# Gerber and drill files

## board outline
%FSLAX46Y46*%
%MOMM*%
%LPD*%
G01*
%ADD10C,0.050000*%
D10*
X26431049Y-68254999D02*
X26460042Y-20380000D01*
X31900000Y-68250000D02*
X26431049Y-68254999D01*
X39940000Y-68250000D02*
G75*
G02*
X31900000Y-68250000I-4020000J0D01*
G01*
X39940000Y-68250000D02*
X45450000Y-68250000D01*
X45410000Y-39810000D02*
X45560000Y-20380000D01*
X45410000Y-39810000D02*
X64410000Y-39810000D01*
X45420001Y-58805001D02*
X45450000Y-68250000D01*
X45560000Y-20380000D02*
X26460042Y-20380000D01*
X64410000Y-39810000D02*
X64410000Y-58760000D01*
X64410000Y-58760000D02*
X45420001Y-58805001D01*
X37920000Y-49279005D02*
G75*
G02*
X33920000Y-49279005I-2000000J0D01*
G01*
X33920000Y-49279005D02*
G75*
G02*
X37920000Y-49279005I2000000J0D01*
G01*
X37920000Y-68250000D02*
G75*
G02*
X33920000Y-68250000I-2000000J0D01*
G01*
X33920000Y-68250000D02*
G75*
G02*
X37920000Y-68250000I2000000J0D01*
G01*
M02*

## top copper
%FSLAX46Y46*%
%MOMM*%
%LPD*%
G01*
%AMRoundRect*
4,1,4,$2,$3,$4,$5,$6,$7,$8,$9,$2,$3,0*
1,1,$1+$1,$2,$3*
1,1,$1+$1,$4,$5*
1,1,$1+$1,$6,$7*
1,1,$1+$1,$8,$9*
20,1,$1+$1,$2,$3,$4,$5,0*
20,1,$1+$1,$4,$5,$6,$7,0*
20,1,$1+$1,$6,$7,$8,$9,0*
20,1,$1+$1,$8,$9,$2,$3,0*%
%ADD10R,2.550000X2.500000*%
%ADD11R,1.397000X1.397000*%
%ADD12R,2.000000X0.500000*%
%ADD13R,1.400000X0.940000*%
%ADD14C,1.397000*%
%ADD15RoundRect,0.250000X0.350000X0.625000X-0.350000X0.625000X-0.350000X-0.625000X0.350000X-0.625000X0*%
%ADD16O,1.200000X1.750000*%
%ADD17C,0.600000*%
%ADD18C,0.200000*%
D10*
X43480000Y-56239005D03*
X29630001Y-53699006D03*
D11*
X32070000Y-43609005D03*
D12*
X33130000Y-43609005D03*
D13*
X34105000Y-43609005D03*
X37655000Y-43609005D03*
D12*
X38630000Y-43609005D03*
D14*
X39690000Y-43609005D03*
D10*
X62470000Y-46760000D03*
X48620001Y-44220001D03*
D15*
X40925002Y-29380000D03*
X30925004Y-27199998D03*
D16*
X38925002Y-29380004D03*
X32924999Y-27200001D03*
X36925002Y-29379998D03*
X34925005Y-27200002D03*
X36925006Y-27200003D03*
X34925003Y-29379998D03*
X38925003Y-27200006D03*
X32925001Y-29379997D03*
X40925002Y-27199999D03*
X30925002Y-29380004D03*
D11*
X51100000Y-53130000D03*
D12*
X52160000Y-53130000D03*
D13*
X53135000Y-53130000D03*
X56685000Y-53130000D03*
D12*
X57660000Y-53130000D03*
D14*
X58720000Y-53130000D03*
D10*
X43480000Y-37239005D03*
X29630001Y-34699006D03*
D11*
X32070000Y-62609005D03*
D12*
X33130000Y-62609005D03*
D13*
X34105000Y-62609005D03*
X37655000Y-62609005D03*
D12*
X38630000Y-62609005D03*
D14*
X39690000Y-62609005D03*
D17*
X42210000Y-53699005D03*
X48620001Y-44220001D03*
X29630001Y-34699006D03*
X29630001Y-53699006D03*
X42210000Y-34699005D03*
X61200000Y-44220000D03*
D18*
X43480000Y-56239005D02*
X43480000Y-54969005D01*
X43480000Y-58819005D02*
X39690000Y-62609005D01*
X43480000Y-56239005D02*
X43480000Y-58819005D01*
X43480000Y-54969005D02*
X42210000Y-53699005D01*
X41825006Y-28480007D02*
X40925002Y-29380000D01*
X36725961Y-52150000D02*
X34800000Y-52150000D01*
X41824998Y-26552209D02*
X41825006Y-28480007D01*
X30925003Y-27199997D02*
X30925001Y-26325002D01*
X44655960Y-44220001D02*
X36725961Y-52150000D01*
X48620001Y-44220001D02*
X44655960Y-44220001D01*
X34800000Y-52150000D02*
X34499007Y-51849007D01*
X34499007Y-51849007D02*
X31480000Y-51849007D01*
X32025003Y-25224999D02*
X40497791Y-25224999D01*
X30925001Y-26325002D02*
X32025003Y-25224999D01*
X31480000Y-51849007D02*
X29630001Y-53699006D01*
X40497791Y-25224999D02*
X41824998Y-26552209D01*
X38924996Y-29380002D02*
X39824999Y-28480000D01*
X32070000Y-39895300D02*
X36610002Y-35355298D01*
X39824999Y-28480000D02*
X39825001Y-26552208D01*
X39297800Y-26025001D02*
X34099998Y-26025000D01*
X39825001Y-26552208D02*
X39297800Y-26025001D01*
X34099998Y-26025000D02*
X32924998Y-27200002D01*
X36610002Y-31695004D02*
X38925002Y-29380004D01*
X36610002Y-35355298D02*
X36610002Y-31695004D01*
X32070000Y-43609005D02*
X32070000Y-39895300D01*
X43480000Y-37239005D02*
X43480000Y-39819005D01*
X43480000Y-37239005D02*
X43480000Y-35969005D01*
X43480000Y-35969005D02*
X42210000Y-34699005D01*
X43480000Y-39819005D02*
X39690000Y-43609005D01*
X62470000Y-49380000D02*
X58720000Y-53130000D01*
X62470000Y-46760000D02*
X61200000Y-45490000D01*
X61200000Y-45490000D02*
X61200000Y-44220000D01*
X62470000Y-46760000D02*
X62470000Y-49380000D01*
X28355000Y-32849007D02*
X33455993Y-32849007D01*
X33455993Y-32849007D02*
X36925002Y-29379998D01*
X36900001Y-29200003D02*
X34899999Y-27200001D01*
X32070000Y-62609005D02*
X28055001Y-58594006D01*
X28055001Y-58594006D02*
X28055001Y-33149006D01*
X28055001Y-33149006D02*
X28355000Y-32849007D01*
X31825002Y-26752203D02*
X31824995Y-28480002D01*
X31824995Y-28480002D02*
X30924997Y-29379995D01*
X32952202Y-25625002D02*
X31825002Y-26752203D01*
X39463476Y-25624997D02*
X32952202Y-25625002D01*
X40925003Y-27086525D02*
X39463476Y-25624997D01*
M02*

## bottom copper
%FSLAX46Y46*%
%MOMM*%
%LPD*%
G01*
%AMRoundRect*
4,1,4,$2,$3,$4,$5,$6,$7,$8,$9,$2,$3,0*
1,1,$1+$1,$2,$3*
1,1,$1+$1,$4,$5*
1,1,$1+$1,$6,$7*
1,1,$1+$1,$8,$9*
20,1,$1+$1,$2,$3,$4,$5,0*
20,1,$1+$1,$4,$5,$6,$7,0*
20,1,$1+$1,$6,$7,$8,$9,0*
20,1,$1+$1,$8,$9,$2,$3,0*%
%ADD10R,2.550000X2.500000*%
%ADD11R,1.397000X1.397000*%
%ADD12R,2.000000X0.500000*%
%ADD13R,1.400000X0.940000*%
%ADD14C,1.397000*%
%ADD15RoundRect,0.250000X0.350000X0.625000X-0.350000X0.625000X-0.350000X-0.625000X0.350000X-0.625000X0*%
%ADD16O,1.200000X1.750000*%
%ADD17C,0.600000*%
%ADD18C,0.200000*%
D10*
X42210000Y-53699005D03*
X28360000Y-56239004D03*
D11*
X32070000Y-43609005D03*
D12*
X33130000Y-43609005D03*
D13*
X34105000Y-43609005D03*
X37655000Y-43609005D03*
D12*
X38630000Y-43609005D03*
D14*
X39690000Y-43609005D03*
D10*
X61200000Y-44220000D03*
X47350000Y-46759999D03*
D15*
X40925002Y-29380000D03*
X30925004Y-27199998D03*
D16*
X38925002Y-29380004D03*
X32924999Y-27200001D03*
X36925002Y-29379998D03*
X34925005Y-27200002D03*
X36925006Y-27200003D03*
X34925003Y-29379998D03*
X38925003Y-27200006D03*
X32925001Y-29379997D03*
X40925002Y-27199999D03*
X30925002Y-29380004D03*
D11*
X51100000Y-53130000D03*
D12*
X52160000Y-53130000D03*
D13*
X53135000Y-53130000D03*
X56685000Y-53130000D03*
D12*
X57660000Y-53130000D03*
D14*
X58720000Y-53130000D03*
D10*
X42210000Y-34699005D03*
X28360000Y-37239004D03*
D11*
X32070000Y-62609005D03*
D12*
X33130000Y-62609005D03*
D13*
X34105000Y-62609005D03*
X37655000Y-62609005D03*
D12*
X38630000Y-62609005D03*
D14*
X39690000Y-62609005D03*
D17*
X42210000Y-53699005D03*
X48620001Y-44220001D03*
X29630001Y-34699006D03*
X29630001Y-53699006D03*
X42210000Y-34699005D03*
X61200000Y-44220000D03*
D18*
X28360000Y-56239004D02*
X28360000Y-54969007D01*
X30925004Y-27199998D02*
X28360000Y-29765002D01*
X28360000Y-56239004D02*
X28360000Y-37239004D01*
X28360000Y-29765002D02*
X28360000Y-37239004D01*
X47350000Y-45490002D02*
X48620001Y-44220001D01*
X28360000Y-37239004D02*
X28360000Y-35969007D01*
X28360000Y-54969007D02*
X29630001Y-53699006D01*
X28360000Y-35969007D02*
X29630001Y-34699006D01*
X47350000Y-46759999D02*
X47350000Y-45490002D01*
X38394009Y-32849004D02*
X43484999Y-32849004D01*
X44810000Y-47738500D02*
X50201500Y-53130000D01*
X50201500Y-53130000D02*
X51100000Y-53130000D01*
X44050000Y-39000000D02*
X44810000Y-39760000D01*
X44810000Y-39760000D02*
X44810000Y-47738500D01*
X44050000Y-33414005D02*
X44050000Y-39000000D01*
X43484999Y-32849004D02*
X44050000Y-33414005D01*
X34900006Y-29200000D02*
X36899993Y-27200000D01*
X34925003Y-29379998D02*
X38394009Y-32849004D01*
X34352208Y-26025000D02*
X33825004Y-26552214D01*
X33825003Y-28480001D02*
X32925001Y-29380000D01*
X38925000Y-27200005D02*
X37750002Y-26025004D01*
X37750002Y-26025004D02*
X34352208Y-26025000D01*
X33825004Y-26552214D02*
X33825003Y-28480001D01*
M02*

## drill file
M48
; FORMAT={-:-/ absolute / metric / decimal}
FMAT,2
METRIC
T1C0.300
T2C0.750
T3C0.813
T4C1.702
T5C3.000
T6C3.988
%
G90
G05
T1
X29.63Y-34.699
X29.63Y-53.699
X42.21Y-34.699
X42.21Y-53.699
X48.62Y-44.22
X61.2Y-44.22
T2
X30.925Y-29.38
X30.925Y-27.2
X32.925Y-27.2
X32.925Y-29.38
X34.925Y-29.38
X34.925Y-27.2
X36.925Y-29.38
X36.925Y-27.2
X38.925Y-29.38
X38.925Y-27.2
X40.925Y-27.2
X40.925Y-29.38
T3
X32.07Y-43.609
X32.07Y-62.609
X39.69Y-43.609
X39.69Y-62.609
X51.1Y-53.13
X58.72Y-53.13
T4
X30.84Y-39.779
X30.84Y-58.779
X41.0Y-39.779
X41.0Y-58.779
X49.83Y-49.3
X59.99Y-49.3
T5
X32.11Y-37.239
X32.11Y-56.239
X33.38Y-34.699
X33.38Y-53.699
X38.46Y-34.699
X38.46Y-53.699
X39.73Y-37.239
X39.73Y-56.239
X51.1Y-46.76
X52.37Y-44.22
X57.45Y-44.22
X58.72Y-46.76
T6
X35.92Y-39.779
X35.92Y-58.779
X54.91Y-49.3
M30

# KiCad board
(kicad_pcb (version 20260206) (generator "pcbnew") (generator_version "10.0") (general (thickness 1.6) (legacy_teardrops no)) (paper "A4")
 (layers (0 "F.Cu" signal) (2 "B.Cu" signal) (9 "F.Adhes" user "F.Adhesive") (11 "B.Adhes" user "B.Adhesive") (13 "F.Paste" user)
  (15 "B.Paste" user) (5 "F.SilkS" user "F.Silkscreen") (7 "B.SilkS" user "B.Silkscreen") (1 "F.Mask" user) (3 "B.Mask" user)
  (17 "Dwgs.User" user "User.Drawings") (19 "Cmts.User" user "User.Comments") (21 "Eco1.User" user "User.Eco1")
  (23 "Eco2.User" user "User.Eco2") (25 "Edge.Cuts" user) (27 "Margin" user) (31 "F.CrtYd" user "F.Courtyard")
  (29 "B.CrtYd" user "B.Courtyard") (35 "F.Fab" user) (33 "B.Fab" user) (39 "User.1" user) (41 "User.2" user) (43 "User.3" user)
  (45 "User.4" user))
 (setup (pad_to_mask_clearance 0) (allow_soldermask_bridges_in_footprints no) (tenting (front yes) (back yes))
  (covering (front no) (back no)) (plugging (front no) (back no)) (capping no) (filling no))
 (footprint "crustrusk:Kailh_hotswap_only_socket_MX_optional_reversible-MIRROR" (layer "F.Cu") (at 35.92 58.779005)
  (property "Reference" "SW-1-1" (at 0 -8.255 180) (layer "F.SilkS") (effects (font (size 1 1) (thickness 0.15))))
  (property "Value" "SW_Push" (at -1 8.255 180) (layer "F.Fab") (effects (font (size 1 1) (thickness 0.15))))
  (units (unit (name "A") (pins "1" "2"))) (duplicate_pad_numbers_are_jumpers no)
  (pad "" np_thru_hole circle (at -5.08 0) (size 1.7018 1.7018) (drill 1.7018) (layers "*.Cu" "*.Mask"))
  (pad "" np_thru_hole circle (at -3.81 -2.54 180) (size 3 3) (drill 3) (layers "*.Cu" "*.Mask"))
  (pad "" np_thru_hole circle (at -2.54 -5.079998) (size 3 3) (drill 3) (layers "*.Cu" "*.Mask"))
  (pad "" np_thru_hole circle (at 0 0) (size 3.9878 3.9878) (drill 3.9878) (layers "*.Cu" "*.Mask"))
  (pad "" np_thru_hole circle (at 2.540002 -5.080001 180) (size 3 3) (drill 3) (layers "*.Cu" "*.Mask"))
  (pad "" np_thru_hole circle (at 3.81 -2.54) (size 3 3) (drill 3) (layers "*.Cu" "*.Mask"))
  (pad "" np_thru_hole circle (at 5.08 0) (size 1.7018 1.7018) (drill 1.7018) (layers "*.Cu" "*.Mask"))
  (pad "1" smd rect (at 6.29 -5.08 180) (size 2.55 2.5) (layers "B.Cu" "B.Mask" "B.Paste") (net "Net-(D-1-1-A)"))
  (pad "1" smd rect (at 7.56 -2.54) (size 2.55 2.5) (layers "F.Cu" "F.Mask" "F.Paste") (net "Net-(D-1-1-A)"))
  (pad "2" smd rect (at -7.56 -2.540001 180) (size 2.55 2.5) (layers "B.Cu" "B.Mask" "B.Paste") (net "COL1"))
  (pad "2" smd rect (at -6.289999 -5.079999) (size 2.55 2.5) (layers "F.Cu" "F.Mask" "F.Paste") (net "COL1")))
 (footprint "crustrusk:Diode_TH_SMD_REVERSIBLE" (layer "F.Cu") (at 35.88 43.609005)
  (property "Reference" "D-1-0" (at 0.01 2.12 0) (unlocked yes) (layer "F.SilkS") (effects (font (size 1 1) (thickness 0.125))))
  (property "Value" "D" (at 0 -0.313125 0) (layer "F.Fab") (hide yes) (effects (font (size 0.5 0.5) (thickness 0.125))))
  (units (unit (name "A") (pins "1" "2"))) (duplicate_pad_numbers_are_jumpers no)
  (pad "1" thru_hole rect (at -3.81 0) (size 1.397 1.397) (drill 0.8128) (layers "*.Cu" "*.Mask") (remove_unused_layers no) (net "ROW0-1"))
  (pad "1" smd rect (at -2.75 0 180) (size 2 0.5) (layers "F.Cu") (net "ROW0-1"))
  (pad "1" smd rect (at -2.75 0) (size 2 0.5) (layers "B.Cu") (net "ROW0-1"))
  (pad "1" smd rect (at -1.775 0 180) (size 1.4 0.94) (layers "F.Cu" "F.Mask" "F.Paste") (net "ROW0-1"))
  (pad "1" smd rect (at -1.775 0) (size 1.4 0.94) (layers "B.Cu" "B.Mask" "B.Paste") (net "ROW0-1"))
  (pad "2" smd rect (at 1.775 0 180) (size 1.4 0.94) (layers "F.Cu" "F.Mask" "F.Paste") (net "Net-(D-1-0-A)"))
  (pad "2" smd rect (at 1.775 0) (size 1.4 0.94) (layers "B.Cu" "B.Mask" "B.Paste") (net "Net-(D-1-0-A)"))
  (pad "2" smd rect (at 2.75 0 180) (size 2 0.5) (layers "F.Cu") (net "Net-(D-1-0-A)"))
  (pad "2" smd rect (at 2.75 0) (size 2 0.5) (layers "B.Cu") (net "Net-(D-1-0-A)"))
  (pad "2" thru_hole circle (at 3.81 0) (size 1.397 1.397) (drill 0.8128) (layers "*.Cu" "*.Mask") (remove_unused_layers no)
   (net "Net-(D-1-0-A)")))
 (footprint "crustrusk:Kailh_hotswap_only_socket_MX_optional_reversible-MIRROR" (layer "F.Cu") (at 54.91 49.3)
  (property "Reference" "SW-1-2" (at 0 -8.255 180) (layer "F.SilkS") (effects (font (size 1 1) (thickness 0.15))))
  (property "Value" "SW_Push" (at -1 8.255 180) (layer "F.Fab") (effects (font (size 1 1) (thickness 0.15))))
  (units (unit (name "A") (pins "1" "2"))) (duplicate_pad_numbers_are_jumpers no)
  (pad "" np_thru_hole circle (at -5.08 0) (size 1.7018 1.7018) (drill 1.7018) (layers "*.Cu" "*.Mask"))
  (pad "" np_thru_hole circle (at -3.81 -2.54 180) (size 3 3) (drill 3) (layers "*.Cu" "*.Mask"))
  (pad "" np_thru_hole circle (at -2.54 -5.079998) (size 3 3) (drill 3) (layers "*.Cu" "*.Mask"))
  (pad "" np_thru_hole circle (at 0 0) (size 3.9878 3.9878) (drill 3.9878) (layers "*.Cu" "*.Mask"))
  (pad "" np_thru_hole circle (at 2.540002 -5.080001 180) (size 3 3) (drill 3) (layers "*.Cu" "*.Mask"))
  (pad "" np_thru_hole circle (at 3.81 -2.54) (size 3 3) (drill 3) (layers "*.Cu" "*.Mask"))
  (pad "" np_thru_hole circle (at 5.08 0) (size 1.7018 1.7018) (drill 1.7018) (layers "*.Cu" "*.Mask"))
  (pad "1" smd rect (at 6.29 -5.08 180) (size 2.55 2.5) (layers "B.Cu" "B.Mask" "B.Paste") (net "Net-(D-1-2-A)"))
  (pad "1" smd rect (at 7.56 -2.54) (size 2.55 2.5) (layers "F.Cu" "F.Mask" "F.Paste") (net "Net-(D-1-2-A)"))
  (pad "2" smd rect (at -7.56 -2.540001 180) (size 2.55 2.5) (layers "B.Cu" "B.Mask" "B.Paste") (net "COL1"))
  (pad "2" smd rect (at -6.289999 -5.079999) (size 2.55 2.5) (layers "F.Cu" "F.Mask" "F.Paste") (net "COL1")))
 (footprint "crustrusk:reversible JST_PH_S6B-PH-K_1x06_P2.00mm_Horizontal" (layer "F.Cu") (at 40.925002 29.38 180)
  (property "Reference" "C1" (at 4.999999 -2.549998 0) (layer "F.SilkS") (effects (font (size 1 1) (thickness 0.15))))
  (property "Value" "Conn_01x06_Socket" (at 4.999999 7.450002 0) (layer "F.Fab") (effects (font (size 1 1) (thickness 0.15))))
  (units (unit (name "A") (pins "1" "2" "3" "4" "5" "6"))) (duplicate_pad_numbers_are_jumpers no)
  (pad "1" thru_hole roundrect (at 0 0 180) (size 1.2 1.75) (drill 0.75) (layers "*.Cu" "*.Mask") (remove_unused_layers no)
   (roundrect_rratio 0.208333) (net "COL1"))
  (pad "1" thru_hole roundrect (at 9.999998 2.180002 180) (size 1.2 1.75) (drill 0.75) (layers "*.Cu" "*.Mask") (remove_unused_layers no)
   (roundrect_rratio 0.208333) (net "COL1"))
  (pad "2" thru_hole oval (at 2 -0.000004 180) (size 1.2 1.75) (drill 0.75) (layers "*.Cu" "*.Mask") (remove_unused_layers no)
   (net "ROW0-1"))
  (pad "2" thru_hole oval (at 8.000003 2.179999 180) (size 1.2 1.75) (drill 0.75) (layers "*.Cu" "*.Mask") (remove_unused_layers no)
   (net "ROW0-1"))
  (pad "3" thru_hole oval (at 4 0.000002 180) (size 1.2 1.75) (drill 0.75) (layers "*.Cu" "*.Mask") (remove_unused_layers no) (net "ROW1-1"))
  (pad "3" thru_hole oval (at 5.999997 2.179998 180) (size 1.2 1.75) (drill 0.75) (layers "*.Cu" "*.Mask") (remove_unused_layers no)
   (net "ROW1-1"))
  (pad "4" thru_hole oval (at 3.999996 2.179997 180) (size 1.2 1.75) (drill 0.75) (layers "*.Cu" "*.Mask") (remove_unused_layers no)
   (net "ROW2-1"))
  (pad "4" thru_hole oval (at 5.999999 0.000002 180) (size 1.2 1.75) (drill 0.75) (layers "*.Cu" "*.Mask") (remove_unused_layers no)
   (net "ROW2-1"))
  (pad "5" thru_hole oval (at 1.999999 2.179994 180) (size 1.2 1.75) (drill 0.75) (layers "*.Cu" "*.Mask") (remove_unused_layers no)
   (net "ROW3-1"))
  (pad "5" thru_hole oval (at 8.000001 0.000003 180) (size 1.2 1.75) (drill 0.75) (layers "*.Cu" "*.Mask") (remove_unused_layers no)
   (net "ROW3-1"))
  (pad "6" thru_hole oval (at 0 2.180001 180) (size 1.2 1.75) (drill 0.75) (layers "*.Cu" "*.Mask") (remove_unused_layers no) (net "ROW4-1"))
  (pad "6" thru_hole oval (at 10 -0.000004 180) (size 1.2 1.75) (drill 0.75) (layers "*.Cu" "*.Mask") (remove_unused_layers no)
   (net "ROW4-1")))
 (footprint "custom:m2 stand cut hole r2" (layer "F.Cu") (at 35.92 49.279005)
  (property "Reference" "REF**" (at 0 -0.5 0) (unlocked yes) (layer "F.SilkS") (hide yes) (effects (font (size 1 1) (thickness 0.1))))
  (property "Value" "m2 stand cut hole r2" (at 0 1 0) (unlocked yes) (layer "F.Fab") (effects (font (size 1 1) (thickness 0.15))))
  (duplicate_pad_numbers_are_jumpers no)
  (fp_circle (center 0 0) (end 2 0) (stroke (width 0.05) (type default)) (fill no) (layer "Edge.Cuts")))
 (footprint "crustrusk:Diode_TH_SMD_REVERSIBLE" (layer "F.Cu") (at 54.91 53.13)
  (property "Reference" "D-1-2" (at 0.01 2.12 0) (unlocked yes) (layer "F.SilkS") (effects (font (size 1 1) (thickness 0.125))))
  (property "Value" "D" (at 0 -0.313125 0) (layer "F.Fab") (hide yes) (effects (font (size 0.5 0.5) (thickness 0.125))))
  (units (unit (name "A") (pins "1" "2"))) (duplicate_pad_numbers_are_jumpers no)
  (pad "1" thru_hole rect (at -3.81 0) (size 1.397 1.397) (drill 0.8128) (layers "*.Cu" "*.Mask") (remove_unused_layers no) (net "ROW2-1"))
  (pad "1" smd rect (at -2.75 0 180) (size 2 0.5) (layers "F.Cu") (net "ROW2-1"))
  (pad "1" smd rect (at -2.75 0) (size 2 0.5) (layers "B.Cu") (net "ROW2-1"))
  (pad "1" smd rect (at -1.775 0 180) (size 1.4 0.94) (layers "F.Cu" "F.Mask" "F.Paste") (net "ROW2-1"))
  (pad "1" smd rect (at -1.775 0) (size 1.4 0.94) (layers "B.Cu" "B.Mask" "B.Paste") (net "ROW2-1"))
  (pad "2" smd rect (at 1.775 0 180) (size 1.4 0.94) (layers "F.Cu" "F.Mask" "F.Paste") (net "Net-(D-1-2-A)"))
  (pad "2" smd rect (at 1.775 0) (size 1.4 0.94) (layers "B.Cu" "B.Mask" "B.Paste") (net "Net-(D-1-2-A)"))
  (pad "2" smd rect (at 2.75 0 180) (size 2 0.5) (layers "F.Cu") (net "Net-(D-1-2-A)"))
  (pad "2" smd rect (at 2.75 0) (size 2 0.5) (layers "B.Cu") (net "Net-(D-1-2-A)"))
  (pad "2" thru_hole circle (at 3.81 0) (size 1.397 1.397) (drill 0.8128) (layers "*.Cu" "*.Mask") (remove_unused_layers no)
   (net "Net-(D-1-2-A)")))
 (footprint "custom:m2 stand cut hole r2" (layer "F.Cu") (at 35.92 68.25)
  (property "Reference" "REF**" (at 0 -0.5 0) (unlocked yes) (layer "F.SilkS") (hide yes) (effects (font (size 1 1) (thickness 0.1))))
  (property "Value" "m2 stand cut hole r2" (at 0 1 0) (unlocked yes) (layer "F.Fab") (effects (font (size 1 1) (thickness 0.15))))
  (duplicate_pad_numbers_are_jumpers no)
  (fp_circle (center 0 0) (end 2 0) (stroke (width 0.05) (type default)) (fill no) (layer "Edge.Cuts")))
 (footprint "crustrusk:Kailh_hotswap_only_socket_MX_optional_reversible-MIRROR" (layer "F.Cu") (at 35.92 39.779005)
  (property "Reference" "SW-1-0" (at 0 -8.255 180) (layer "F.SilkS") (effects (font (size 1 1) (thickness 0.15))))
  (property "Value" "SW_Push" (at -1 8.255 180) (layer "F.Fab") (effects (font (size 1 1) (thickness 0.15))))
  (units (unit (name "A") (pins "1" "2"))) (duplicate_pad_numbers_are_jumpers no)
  (pad "" np_thru_hole circle (at -5.08 0) (size 1.7018 1.7018) (drill 1.7018) (layers "*.Cu" "*.Mask"))
  (pad "" np_thru_hole circle (at -3.81 -2.54 180) (size 3 3) (drill 3) (layers "*.Cu" "*.Mask"))
  (pad "" np_thru_hole circle (at -2.54 -5.079998) (size 3 3) (drill 3) (layers "*.Cu" "*.Mask"))
  (pad "" np_thru_hole circle (at 0 0) (size 3.9878 3.9878) (drill 3.9878) (layers "*.Cu" "*.Mask"))
  (pad "" np_thru_hole circle (at 2.540002 -5.080001 180) (size 3 3) (drill 3) (layers "*.Cu" "*.Mask"))
  (pad "" np_thru_hole circle (at 3.81 -2.54) (size 3 3) (drill 3) (layers "*.Cu" "*.Mask"))
  (pad "" np_thru_hole circle (at 5.08 0) (size 1.7018 1.7018) (drill 1.7018) (layers "*.Cu" "*.Mask"))
  (pad "1" smd rect (at 6.29 -5.08 180) (size 2.55 2.5) (layers "B.Cu" "B.Mask" "B.Paste") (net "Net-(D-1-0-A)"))
  (pad "1" smd rect (at 7.56 -2.54) (size 2.55 2.5) (layers "F.Cu" "F.Mask" "F.Paste") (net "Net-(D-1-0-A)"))
  (pad "2" smd rect (at -7.56 -2.540001 180) (size 2.55 2.5) (layers "B.Cu" "B.Mask" "B.Paste") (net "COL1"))
  (pad "2" smd rect (at -6.289999 -5.079999) (size 2.55 2.5) (layers "F.Cu" "F.Mask" "F.Paste") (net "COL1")))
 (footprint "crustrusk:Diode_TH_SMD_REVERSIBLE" (layer "F.Cu") (at 35.88 62.609005)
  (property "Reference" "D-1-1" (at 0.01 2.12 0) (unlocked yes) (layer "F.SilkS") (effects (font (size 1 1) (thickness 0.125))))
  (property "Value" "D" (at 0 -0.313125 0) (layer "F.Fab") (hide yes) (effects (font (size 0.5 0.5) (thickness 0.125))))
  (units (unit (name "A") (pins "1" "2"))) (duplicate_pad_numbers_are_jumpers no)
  (pad "1" thru_hole rect (at -3.81 0) (size 1.397 1.397) (drill 0.8128) (layers "*.Cu" "*.Mask") (remove_unused_layers no) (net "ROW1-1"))
  (pad "1" smd rect (at -2.75 0 180) (size 2 0.5) (layers "F.Cu") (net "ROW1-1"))
  (pad "1" smd rect (at -2.75 0) (size 2 0.5) (layers "B.Cu") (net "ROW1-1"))
  (pad "1" smd rect (at -1.775 0 180) (size 1.4 0.94) (layers "F.Cu" "F.Mask" "F.Paste") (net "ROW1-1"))
  (pad "1" smd rect (at -1.775 0) (size 1.4 0.94) (layers "B.Cu" "B.Mask" "B.Paste") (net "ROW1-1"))
  (pad "2" smd rect (at 1.775 0 180) (size 1.4 0.94) (layers "F.Cu" "F.Mask" "F.Paste") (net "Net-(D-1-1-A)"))
  (pad "2" smd rect (at 1.775 0) (size 1.4 0.94) (layers "B.Cu" "B.Mask" "B.Paste") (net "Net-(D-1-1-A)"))
  (pad "2" smd rect (at 2.75 0 180) (size 2 0.5) (layers "F.Cu") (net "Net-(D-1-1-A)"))
  (pad "2" smd rect (at 2.75 0) (size 2 0.5) (layers "B.Cu") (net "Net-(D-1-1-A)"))
  (pad "2" thru_hole circle (at 3.81 0) (size 1.397 1.397) (drill 0.8128) (layers "*.Cu" "*.Mask") (remove_unused_layers no)
   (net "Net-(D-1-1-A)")))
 (gr_line (start 26.431049 68.254999) (end 26.460042 20.38) (stroke (width 0.05) (type default)) (layer "Edge.Cuts"))
 (gr_line (start 31.9 68.25) (end 26.431049 68.254999) (stroke (width 0.05) (type default)) (layer "Edge.Cuts"))
 (gr_arc (start 39.94 68.25) (mid 35.92 72.27) (end 31.9 68.25) (stroke (width 0.05) (type default)) (layer "Edge.Cuts"))
 (gr_line (start 39.94 68.25) (end 45.45 68.25) (stroke (width 0.05) (type default)) (layer "Edge.Cuts"))
 (gr_line (start 45.41 39.81) (end 45.56 20.38) (stroke (width 0.05) (type default)) (layer "Edge.Cuts"))
 (gr_line (start 45.41 39.81) (end 64.41 39.81) (stroke (width 0.05) (type default)) (layer "Edge.Cuts"))
 (gr_line (start 45.420001 58.805001) (end 45.45 68.25) (stroke (width 0.05) (type default)) (layer "Edge.Cuts"))
 (gr_line (start 45.56 20.38) (end 26.460042 20.38) (stroke (width 0.05) (type default)) (layer "Edge.Cuts"))
 (gr_line (start 64.41 39.81) (end 64.41 58.76) (stroke (width 0.05) (type default)) (layer "Edge.Cuts"))
 (gr_line (start 64.41 58.76) (end 45.420001 58.805001) (stroke (width 0.05) (type default)) (layer "Edge.Cuts"))
 (segment (start 43.48 56.239005) (end 43.48 54.969005) (width 0.2) (layer "F.Cu") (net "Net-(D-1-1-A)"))
 (segment (start 43.48 58.819005) (end 39.69 62.609005) (width 0.2) (layer "F.Cu") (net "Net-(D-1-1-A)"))
 (segment (start 43.48 56.239005) (end 43.48 58.819005) (width 0.2) (layer "F.Cu") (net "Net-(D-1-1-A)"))
 (segment (start 43.48 54.969005) (end 42.21 53.699005) (width 0.2) (layer "F.Cu") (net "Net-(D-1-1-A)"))
 (via (at 42.21 53.699005) (size 0.6) (drill 0.3) (layers "F.Cu" "B.Cu") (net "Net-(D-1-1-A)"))
 (segment (start 41.825006 28.480007) (end 40.925002 29.38) (width 0.2) (layer "F.Cu") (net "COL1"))
 (segment (start 36.725961 52.15) (end 34.8 52.15) (width 0.2) (layer "F.Cu") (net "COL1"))
 (segment (start 41.824998 26.552209) (end 41.825006 28.480007) (width 0.2) (layer "F.Cu") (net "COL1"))
 (segment (start 30.925003 27.199997) (end 30.925001 26.325002) (width 0.2) (layer "F.Cu") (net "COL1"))
 (segment (start 44.65596 44.220001) (end 36.725961 52.15) (width 0.2) (layer "F.Cu") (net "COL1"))
 (segment (start 48.620001 44.220001) (end 44.65596 44.220001) (width 0.2) (layer "F.Cu") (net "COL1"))
 (segment (start 34.8 52.15) (end 34.499007 51.849007) (width 0.2) (layer "F.Cu") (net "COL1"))
 (segment (start 34.499007 51.849007) (end 31.48 51.849007) (width 0.2) (layer "F.Cu") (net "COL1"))
 (segment (start 32.025003 25.224999) (end 40.497791 25.224999) (width 0.2) (layer "F.Cu") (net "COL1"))
 (segment (start 30.925001 26.325002) (end 32.025003 25.224999) (width 0.2) (layer "F.Cu") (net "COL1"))
 (segment (start 31.48 51.849007) (end 29.630001 53.699006) (width 0.2) (layer "F.Cu") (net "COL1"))
 (segment (start 40.497791 25.224999) (end 41.824998 26.552209) (width 0.2) (layer "F.Cu") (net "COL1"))
 (via (at 48.620001 44.220001) (size 0.6) (drill 0.3) (layers "F.Cu" "B.Cu") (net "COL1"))
 (via (at 29.630001 34.699006) (size 0.6) (drill 0.3) (layers "F.Cu" "B.Cu") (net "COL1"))
 (via (at 29.630001 53.699006) (size 0.6) (drill 0.3) (layers "F.Cu" "B.Cu") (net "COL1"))
 (segment (start 28.36 56.239004) (end 28.36 54.969007) (width 0.2) (layer "B.Cu") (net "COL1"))
 (segment (start 30.925004 27.199998) (end 28.36 29.765002) (width 0.2) (layer "B.Cu") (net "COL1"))
 (segment (start 28.36 56.239004) (end 28.36 37.239004) (width 0.2) (layer "B.Cu") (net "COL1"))
 (segment (start 28.36 29.765002) (end 28.36 37.239004) (width 0.2) (layer "B.Cu") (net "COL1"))
 (segment (start 47.35 45.490002) (end 48.620001 44.220001) (width 0.2) (layer "B.Cu") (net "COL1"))
 (segment (start 28.36 37.239004) (end 28.36 35.969007) (width 0.2) (layer "B.Cu") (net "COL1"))
 (segment (start 28.36 54.969007) (end 29.630001 53.699006) (width 0.2) (layer "B.Cu") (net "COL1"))
 (segment (start 28.36 35.969007) (end 29.630001 34.699006) (width 0.2) (layer "B.Cu") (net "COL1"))
 (segment (start 47.35 46.759999) (end 47.35 45.490002) (width 0.2) (layer "B.Cu") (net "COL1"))
 (segment (start 38.924996 29.380002) (end 39.824999 28.48) (width 0.2) (layer "F.Cu") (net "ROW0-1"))
 (segment (start 32.07 39.8953) (end 36.610002 35.355298) (width 0.2) (layer "F.Cu") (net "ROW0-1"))
 (segment (start 39.824999 28.48) (end 39.825001 26.552208) (width 0.2) (layer "F.Cu") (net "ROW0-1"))
 (segment (start 39.2978 26.025001) (end 34.099998 26.025) (width 0.2) (layer "F.Cu") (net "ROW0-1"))
 (segment (start 39.825001 26.552208) (end 39.2978 26.025001) (width 0.2) (layer "F.Cu") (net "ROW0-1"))
 (segment (start 34.099998 26.025) (end 32.924998 27.200002) (width 0.2) (layer "F.Cu") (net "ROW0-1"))
 (segment (start 36.610002 31.695004) (end 38.925002 29.380004) (width 0.2) (layer "F.Cu") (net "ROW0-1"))
 (segment (start 36.610002 35.355298) (end 36.610002 31.695004) (width 0.2) (layer "F.Cu") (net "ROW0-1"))
 (segment (start 32.07 43.609005) (end 32.07 39.8953) (width 0.2) (layer "F.Cu") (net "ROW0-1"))
 (segment (start 43.48 37.239005) (end 43.48 39.819005) (width 0.2) (layer "F.Cu") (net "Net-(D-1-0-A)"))
 (segment (start 43.48 37.239005) (end 43.48 35.969005) (width 0.2) (layer "F.Cu") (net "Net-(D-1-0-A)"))
 (segment (start 43.48 35.969005) (end 42.21 34.699005) (width 0.2) (layer "F.Cu") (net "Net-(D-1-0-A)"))
 (segment (start 43.48 39.819005) (end 39.69 43.609005) (width 0.2) (layer "F.Cu") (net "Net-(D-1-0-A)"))
 (via (at 42.21 34.699005) (size 0.6) (drill 0.3) (layers "F.Cu" "B.Cu") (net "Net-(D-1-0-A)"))
 (segment (start 62.47 49.38) (end 58.72 53.13) (width 0.2) (layer "F.Cu") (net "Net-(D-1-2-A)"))
 (segment (start 62.47 46.76) (end 61.2 45.49) (width 0.2) (layer "F.Cu") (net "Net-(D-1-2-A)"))
 (segment (start 61.2 45.49) (end 61.2 44.22) (width 0.2) (layer "F.Cu") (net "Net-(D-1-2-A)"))
 (segment (start 62.47 46.76) (end 62.47 49.38) (width 0.2) (layer "F.Cu") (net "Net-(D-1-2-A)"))
 (via (at 61.2 44.22) (size 0.6) (drill 0.3) (layers "F.Cu" "B.Cu") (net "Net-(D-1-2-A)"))
 (segment (start 28.355 32.849007) (end 33.455993 32.849007) (width 0.2) (layer "F.Cu") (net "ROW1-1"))
 (segment (start 33.455993 32.849007) (end 36.925002 29.379998) (width 0.2) (layer "F.Cu") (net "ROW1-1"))
 (segment (start 36.900001 29.200003) (end 34.899999 27.200001) (width 0.2) (layer "F.Cu") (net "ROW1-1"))
 (segment (start 32.07 62.609005) (end 28.055001 58.594006) (width 0.2) (layer "F.Cu") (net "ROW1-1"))
 (segment (start 28.055001 58.594006) (end 28.055001 33.149006) (width 0.2) (layer "F.Cu") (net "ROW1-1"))
 (segment (start 28.055001 33.149006) (end 28.355 32.849007) (width 0.2) (layer "F.Cu") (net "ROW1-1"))
 (segment (start 38.394009 32.849004) (end 43.484999 32.849004) (width 0.2) (layer "B.Cu") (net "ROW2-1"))
 (segment (start 44.81 47.7385) (end 50.2015 53.13) (width 0.2) (layer "B.Cu") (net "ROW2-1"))
 (segment (start 50.2015 53.13) (end 51.1 53.13) (width 0.2) (layer "B.Cu") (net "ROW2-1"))
 (segment (start 44.05 39) (end 44.81 39.76) (width 0.2) (layer "B.Cu") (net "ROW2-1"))
 (segment (start 44.81 39.76) (end 44.81 47.7385) (width 0.2) (layer "B.Cu") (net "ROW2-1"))
 (segment (start 44.05 33.414005) (end 44.05 39) (width 0.2) (layer "B.Cu") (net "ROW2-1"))
 (segment (start 43.484999 32.849004) (end 44.05 33.414005) (width 0.2) (layer "B.Cu") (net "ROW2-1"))
 (segment (start 34.900006 29.2) (end 36.899993 27.2) (width 0.2) (layer "B.Cu") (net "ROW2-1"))
 (segment (start 34.925003 29.379998) (end 38.394009 32.849004) (width 0.2) (layer "B.Cu") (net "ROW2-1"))
 (segment (start 34.352208 26.025) (end 33.825004 26.552214) (width 0.2) (layer "B.Cu") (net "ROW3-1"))
 (segment (start 33.825003 28.480001) (end 32.925001 29.38) (width 0.2) (layer "B.Cu") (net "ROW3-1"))
 (segment (start 38.925 27.200005) (end 37.750002 26.025004) (width 0.2) (layer "B.Cu") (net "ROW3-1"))
 (segment (start 37.750002 26.025004) (end 34.352208 26.025) (width 0.2) (layer "B.Cu") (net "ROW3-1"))
 (segment (start 33.825004 26.552214) (end 33.825003 28.480001) (width 0.2) (layer "B.Cu") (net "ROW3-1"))
 (segment (start 31.825002 26.752203) (end 31.824995 28.480002) (width 0.2) (layer "F.Cu") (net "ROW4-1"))
 (segment (start 31.824995 28.480002) (end 30.924997 29.379995) (width 0.2) (layer "F.Cu") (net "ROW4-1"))
 (segment (start 32.952202 25.625002) (end 31.825002 26.752203) (width 0.2) (layer "F.Cu") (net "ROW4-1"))
 (segment (start 39.463476 25.624997) (end 32.952202 25.625002) (width 0.2) (layer "F.Cu") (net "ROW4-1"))
 (segment (start 40.925003 27.086525) (end 39.463476 25.624997) (width 0.2) (layer "F.Cu") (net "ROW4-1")))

